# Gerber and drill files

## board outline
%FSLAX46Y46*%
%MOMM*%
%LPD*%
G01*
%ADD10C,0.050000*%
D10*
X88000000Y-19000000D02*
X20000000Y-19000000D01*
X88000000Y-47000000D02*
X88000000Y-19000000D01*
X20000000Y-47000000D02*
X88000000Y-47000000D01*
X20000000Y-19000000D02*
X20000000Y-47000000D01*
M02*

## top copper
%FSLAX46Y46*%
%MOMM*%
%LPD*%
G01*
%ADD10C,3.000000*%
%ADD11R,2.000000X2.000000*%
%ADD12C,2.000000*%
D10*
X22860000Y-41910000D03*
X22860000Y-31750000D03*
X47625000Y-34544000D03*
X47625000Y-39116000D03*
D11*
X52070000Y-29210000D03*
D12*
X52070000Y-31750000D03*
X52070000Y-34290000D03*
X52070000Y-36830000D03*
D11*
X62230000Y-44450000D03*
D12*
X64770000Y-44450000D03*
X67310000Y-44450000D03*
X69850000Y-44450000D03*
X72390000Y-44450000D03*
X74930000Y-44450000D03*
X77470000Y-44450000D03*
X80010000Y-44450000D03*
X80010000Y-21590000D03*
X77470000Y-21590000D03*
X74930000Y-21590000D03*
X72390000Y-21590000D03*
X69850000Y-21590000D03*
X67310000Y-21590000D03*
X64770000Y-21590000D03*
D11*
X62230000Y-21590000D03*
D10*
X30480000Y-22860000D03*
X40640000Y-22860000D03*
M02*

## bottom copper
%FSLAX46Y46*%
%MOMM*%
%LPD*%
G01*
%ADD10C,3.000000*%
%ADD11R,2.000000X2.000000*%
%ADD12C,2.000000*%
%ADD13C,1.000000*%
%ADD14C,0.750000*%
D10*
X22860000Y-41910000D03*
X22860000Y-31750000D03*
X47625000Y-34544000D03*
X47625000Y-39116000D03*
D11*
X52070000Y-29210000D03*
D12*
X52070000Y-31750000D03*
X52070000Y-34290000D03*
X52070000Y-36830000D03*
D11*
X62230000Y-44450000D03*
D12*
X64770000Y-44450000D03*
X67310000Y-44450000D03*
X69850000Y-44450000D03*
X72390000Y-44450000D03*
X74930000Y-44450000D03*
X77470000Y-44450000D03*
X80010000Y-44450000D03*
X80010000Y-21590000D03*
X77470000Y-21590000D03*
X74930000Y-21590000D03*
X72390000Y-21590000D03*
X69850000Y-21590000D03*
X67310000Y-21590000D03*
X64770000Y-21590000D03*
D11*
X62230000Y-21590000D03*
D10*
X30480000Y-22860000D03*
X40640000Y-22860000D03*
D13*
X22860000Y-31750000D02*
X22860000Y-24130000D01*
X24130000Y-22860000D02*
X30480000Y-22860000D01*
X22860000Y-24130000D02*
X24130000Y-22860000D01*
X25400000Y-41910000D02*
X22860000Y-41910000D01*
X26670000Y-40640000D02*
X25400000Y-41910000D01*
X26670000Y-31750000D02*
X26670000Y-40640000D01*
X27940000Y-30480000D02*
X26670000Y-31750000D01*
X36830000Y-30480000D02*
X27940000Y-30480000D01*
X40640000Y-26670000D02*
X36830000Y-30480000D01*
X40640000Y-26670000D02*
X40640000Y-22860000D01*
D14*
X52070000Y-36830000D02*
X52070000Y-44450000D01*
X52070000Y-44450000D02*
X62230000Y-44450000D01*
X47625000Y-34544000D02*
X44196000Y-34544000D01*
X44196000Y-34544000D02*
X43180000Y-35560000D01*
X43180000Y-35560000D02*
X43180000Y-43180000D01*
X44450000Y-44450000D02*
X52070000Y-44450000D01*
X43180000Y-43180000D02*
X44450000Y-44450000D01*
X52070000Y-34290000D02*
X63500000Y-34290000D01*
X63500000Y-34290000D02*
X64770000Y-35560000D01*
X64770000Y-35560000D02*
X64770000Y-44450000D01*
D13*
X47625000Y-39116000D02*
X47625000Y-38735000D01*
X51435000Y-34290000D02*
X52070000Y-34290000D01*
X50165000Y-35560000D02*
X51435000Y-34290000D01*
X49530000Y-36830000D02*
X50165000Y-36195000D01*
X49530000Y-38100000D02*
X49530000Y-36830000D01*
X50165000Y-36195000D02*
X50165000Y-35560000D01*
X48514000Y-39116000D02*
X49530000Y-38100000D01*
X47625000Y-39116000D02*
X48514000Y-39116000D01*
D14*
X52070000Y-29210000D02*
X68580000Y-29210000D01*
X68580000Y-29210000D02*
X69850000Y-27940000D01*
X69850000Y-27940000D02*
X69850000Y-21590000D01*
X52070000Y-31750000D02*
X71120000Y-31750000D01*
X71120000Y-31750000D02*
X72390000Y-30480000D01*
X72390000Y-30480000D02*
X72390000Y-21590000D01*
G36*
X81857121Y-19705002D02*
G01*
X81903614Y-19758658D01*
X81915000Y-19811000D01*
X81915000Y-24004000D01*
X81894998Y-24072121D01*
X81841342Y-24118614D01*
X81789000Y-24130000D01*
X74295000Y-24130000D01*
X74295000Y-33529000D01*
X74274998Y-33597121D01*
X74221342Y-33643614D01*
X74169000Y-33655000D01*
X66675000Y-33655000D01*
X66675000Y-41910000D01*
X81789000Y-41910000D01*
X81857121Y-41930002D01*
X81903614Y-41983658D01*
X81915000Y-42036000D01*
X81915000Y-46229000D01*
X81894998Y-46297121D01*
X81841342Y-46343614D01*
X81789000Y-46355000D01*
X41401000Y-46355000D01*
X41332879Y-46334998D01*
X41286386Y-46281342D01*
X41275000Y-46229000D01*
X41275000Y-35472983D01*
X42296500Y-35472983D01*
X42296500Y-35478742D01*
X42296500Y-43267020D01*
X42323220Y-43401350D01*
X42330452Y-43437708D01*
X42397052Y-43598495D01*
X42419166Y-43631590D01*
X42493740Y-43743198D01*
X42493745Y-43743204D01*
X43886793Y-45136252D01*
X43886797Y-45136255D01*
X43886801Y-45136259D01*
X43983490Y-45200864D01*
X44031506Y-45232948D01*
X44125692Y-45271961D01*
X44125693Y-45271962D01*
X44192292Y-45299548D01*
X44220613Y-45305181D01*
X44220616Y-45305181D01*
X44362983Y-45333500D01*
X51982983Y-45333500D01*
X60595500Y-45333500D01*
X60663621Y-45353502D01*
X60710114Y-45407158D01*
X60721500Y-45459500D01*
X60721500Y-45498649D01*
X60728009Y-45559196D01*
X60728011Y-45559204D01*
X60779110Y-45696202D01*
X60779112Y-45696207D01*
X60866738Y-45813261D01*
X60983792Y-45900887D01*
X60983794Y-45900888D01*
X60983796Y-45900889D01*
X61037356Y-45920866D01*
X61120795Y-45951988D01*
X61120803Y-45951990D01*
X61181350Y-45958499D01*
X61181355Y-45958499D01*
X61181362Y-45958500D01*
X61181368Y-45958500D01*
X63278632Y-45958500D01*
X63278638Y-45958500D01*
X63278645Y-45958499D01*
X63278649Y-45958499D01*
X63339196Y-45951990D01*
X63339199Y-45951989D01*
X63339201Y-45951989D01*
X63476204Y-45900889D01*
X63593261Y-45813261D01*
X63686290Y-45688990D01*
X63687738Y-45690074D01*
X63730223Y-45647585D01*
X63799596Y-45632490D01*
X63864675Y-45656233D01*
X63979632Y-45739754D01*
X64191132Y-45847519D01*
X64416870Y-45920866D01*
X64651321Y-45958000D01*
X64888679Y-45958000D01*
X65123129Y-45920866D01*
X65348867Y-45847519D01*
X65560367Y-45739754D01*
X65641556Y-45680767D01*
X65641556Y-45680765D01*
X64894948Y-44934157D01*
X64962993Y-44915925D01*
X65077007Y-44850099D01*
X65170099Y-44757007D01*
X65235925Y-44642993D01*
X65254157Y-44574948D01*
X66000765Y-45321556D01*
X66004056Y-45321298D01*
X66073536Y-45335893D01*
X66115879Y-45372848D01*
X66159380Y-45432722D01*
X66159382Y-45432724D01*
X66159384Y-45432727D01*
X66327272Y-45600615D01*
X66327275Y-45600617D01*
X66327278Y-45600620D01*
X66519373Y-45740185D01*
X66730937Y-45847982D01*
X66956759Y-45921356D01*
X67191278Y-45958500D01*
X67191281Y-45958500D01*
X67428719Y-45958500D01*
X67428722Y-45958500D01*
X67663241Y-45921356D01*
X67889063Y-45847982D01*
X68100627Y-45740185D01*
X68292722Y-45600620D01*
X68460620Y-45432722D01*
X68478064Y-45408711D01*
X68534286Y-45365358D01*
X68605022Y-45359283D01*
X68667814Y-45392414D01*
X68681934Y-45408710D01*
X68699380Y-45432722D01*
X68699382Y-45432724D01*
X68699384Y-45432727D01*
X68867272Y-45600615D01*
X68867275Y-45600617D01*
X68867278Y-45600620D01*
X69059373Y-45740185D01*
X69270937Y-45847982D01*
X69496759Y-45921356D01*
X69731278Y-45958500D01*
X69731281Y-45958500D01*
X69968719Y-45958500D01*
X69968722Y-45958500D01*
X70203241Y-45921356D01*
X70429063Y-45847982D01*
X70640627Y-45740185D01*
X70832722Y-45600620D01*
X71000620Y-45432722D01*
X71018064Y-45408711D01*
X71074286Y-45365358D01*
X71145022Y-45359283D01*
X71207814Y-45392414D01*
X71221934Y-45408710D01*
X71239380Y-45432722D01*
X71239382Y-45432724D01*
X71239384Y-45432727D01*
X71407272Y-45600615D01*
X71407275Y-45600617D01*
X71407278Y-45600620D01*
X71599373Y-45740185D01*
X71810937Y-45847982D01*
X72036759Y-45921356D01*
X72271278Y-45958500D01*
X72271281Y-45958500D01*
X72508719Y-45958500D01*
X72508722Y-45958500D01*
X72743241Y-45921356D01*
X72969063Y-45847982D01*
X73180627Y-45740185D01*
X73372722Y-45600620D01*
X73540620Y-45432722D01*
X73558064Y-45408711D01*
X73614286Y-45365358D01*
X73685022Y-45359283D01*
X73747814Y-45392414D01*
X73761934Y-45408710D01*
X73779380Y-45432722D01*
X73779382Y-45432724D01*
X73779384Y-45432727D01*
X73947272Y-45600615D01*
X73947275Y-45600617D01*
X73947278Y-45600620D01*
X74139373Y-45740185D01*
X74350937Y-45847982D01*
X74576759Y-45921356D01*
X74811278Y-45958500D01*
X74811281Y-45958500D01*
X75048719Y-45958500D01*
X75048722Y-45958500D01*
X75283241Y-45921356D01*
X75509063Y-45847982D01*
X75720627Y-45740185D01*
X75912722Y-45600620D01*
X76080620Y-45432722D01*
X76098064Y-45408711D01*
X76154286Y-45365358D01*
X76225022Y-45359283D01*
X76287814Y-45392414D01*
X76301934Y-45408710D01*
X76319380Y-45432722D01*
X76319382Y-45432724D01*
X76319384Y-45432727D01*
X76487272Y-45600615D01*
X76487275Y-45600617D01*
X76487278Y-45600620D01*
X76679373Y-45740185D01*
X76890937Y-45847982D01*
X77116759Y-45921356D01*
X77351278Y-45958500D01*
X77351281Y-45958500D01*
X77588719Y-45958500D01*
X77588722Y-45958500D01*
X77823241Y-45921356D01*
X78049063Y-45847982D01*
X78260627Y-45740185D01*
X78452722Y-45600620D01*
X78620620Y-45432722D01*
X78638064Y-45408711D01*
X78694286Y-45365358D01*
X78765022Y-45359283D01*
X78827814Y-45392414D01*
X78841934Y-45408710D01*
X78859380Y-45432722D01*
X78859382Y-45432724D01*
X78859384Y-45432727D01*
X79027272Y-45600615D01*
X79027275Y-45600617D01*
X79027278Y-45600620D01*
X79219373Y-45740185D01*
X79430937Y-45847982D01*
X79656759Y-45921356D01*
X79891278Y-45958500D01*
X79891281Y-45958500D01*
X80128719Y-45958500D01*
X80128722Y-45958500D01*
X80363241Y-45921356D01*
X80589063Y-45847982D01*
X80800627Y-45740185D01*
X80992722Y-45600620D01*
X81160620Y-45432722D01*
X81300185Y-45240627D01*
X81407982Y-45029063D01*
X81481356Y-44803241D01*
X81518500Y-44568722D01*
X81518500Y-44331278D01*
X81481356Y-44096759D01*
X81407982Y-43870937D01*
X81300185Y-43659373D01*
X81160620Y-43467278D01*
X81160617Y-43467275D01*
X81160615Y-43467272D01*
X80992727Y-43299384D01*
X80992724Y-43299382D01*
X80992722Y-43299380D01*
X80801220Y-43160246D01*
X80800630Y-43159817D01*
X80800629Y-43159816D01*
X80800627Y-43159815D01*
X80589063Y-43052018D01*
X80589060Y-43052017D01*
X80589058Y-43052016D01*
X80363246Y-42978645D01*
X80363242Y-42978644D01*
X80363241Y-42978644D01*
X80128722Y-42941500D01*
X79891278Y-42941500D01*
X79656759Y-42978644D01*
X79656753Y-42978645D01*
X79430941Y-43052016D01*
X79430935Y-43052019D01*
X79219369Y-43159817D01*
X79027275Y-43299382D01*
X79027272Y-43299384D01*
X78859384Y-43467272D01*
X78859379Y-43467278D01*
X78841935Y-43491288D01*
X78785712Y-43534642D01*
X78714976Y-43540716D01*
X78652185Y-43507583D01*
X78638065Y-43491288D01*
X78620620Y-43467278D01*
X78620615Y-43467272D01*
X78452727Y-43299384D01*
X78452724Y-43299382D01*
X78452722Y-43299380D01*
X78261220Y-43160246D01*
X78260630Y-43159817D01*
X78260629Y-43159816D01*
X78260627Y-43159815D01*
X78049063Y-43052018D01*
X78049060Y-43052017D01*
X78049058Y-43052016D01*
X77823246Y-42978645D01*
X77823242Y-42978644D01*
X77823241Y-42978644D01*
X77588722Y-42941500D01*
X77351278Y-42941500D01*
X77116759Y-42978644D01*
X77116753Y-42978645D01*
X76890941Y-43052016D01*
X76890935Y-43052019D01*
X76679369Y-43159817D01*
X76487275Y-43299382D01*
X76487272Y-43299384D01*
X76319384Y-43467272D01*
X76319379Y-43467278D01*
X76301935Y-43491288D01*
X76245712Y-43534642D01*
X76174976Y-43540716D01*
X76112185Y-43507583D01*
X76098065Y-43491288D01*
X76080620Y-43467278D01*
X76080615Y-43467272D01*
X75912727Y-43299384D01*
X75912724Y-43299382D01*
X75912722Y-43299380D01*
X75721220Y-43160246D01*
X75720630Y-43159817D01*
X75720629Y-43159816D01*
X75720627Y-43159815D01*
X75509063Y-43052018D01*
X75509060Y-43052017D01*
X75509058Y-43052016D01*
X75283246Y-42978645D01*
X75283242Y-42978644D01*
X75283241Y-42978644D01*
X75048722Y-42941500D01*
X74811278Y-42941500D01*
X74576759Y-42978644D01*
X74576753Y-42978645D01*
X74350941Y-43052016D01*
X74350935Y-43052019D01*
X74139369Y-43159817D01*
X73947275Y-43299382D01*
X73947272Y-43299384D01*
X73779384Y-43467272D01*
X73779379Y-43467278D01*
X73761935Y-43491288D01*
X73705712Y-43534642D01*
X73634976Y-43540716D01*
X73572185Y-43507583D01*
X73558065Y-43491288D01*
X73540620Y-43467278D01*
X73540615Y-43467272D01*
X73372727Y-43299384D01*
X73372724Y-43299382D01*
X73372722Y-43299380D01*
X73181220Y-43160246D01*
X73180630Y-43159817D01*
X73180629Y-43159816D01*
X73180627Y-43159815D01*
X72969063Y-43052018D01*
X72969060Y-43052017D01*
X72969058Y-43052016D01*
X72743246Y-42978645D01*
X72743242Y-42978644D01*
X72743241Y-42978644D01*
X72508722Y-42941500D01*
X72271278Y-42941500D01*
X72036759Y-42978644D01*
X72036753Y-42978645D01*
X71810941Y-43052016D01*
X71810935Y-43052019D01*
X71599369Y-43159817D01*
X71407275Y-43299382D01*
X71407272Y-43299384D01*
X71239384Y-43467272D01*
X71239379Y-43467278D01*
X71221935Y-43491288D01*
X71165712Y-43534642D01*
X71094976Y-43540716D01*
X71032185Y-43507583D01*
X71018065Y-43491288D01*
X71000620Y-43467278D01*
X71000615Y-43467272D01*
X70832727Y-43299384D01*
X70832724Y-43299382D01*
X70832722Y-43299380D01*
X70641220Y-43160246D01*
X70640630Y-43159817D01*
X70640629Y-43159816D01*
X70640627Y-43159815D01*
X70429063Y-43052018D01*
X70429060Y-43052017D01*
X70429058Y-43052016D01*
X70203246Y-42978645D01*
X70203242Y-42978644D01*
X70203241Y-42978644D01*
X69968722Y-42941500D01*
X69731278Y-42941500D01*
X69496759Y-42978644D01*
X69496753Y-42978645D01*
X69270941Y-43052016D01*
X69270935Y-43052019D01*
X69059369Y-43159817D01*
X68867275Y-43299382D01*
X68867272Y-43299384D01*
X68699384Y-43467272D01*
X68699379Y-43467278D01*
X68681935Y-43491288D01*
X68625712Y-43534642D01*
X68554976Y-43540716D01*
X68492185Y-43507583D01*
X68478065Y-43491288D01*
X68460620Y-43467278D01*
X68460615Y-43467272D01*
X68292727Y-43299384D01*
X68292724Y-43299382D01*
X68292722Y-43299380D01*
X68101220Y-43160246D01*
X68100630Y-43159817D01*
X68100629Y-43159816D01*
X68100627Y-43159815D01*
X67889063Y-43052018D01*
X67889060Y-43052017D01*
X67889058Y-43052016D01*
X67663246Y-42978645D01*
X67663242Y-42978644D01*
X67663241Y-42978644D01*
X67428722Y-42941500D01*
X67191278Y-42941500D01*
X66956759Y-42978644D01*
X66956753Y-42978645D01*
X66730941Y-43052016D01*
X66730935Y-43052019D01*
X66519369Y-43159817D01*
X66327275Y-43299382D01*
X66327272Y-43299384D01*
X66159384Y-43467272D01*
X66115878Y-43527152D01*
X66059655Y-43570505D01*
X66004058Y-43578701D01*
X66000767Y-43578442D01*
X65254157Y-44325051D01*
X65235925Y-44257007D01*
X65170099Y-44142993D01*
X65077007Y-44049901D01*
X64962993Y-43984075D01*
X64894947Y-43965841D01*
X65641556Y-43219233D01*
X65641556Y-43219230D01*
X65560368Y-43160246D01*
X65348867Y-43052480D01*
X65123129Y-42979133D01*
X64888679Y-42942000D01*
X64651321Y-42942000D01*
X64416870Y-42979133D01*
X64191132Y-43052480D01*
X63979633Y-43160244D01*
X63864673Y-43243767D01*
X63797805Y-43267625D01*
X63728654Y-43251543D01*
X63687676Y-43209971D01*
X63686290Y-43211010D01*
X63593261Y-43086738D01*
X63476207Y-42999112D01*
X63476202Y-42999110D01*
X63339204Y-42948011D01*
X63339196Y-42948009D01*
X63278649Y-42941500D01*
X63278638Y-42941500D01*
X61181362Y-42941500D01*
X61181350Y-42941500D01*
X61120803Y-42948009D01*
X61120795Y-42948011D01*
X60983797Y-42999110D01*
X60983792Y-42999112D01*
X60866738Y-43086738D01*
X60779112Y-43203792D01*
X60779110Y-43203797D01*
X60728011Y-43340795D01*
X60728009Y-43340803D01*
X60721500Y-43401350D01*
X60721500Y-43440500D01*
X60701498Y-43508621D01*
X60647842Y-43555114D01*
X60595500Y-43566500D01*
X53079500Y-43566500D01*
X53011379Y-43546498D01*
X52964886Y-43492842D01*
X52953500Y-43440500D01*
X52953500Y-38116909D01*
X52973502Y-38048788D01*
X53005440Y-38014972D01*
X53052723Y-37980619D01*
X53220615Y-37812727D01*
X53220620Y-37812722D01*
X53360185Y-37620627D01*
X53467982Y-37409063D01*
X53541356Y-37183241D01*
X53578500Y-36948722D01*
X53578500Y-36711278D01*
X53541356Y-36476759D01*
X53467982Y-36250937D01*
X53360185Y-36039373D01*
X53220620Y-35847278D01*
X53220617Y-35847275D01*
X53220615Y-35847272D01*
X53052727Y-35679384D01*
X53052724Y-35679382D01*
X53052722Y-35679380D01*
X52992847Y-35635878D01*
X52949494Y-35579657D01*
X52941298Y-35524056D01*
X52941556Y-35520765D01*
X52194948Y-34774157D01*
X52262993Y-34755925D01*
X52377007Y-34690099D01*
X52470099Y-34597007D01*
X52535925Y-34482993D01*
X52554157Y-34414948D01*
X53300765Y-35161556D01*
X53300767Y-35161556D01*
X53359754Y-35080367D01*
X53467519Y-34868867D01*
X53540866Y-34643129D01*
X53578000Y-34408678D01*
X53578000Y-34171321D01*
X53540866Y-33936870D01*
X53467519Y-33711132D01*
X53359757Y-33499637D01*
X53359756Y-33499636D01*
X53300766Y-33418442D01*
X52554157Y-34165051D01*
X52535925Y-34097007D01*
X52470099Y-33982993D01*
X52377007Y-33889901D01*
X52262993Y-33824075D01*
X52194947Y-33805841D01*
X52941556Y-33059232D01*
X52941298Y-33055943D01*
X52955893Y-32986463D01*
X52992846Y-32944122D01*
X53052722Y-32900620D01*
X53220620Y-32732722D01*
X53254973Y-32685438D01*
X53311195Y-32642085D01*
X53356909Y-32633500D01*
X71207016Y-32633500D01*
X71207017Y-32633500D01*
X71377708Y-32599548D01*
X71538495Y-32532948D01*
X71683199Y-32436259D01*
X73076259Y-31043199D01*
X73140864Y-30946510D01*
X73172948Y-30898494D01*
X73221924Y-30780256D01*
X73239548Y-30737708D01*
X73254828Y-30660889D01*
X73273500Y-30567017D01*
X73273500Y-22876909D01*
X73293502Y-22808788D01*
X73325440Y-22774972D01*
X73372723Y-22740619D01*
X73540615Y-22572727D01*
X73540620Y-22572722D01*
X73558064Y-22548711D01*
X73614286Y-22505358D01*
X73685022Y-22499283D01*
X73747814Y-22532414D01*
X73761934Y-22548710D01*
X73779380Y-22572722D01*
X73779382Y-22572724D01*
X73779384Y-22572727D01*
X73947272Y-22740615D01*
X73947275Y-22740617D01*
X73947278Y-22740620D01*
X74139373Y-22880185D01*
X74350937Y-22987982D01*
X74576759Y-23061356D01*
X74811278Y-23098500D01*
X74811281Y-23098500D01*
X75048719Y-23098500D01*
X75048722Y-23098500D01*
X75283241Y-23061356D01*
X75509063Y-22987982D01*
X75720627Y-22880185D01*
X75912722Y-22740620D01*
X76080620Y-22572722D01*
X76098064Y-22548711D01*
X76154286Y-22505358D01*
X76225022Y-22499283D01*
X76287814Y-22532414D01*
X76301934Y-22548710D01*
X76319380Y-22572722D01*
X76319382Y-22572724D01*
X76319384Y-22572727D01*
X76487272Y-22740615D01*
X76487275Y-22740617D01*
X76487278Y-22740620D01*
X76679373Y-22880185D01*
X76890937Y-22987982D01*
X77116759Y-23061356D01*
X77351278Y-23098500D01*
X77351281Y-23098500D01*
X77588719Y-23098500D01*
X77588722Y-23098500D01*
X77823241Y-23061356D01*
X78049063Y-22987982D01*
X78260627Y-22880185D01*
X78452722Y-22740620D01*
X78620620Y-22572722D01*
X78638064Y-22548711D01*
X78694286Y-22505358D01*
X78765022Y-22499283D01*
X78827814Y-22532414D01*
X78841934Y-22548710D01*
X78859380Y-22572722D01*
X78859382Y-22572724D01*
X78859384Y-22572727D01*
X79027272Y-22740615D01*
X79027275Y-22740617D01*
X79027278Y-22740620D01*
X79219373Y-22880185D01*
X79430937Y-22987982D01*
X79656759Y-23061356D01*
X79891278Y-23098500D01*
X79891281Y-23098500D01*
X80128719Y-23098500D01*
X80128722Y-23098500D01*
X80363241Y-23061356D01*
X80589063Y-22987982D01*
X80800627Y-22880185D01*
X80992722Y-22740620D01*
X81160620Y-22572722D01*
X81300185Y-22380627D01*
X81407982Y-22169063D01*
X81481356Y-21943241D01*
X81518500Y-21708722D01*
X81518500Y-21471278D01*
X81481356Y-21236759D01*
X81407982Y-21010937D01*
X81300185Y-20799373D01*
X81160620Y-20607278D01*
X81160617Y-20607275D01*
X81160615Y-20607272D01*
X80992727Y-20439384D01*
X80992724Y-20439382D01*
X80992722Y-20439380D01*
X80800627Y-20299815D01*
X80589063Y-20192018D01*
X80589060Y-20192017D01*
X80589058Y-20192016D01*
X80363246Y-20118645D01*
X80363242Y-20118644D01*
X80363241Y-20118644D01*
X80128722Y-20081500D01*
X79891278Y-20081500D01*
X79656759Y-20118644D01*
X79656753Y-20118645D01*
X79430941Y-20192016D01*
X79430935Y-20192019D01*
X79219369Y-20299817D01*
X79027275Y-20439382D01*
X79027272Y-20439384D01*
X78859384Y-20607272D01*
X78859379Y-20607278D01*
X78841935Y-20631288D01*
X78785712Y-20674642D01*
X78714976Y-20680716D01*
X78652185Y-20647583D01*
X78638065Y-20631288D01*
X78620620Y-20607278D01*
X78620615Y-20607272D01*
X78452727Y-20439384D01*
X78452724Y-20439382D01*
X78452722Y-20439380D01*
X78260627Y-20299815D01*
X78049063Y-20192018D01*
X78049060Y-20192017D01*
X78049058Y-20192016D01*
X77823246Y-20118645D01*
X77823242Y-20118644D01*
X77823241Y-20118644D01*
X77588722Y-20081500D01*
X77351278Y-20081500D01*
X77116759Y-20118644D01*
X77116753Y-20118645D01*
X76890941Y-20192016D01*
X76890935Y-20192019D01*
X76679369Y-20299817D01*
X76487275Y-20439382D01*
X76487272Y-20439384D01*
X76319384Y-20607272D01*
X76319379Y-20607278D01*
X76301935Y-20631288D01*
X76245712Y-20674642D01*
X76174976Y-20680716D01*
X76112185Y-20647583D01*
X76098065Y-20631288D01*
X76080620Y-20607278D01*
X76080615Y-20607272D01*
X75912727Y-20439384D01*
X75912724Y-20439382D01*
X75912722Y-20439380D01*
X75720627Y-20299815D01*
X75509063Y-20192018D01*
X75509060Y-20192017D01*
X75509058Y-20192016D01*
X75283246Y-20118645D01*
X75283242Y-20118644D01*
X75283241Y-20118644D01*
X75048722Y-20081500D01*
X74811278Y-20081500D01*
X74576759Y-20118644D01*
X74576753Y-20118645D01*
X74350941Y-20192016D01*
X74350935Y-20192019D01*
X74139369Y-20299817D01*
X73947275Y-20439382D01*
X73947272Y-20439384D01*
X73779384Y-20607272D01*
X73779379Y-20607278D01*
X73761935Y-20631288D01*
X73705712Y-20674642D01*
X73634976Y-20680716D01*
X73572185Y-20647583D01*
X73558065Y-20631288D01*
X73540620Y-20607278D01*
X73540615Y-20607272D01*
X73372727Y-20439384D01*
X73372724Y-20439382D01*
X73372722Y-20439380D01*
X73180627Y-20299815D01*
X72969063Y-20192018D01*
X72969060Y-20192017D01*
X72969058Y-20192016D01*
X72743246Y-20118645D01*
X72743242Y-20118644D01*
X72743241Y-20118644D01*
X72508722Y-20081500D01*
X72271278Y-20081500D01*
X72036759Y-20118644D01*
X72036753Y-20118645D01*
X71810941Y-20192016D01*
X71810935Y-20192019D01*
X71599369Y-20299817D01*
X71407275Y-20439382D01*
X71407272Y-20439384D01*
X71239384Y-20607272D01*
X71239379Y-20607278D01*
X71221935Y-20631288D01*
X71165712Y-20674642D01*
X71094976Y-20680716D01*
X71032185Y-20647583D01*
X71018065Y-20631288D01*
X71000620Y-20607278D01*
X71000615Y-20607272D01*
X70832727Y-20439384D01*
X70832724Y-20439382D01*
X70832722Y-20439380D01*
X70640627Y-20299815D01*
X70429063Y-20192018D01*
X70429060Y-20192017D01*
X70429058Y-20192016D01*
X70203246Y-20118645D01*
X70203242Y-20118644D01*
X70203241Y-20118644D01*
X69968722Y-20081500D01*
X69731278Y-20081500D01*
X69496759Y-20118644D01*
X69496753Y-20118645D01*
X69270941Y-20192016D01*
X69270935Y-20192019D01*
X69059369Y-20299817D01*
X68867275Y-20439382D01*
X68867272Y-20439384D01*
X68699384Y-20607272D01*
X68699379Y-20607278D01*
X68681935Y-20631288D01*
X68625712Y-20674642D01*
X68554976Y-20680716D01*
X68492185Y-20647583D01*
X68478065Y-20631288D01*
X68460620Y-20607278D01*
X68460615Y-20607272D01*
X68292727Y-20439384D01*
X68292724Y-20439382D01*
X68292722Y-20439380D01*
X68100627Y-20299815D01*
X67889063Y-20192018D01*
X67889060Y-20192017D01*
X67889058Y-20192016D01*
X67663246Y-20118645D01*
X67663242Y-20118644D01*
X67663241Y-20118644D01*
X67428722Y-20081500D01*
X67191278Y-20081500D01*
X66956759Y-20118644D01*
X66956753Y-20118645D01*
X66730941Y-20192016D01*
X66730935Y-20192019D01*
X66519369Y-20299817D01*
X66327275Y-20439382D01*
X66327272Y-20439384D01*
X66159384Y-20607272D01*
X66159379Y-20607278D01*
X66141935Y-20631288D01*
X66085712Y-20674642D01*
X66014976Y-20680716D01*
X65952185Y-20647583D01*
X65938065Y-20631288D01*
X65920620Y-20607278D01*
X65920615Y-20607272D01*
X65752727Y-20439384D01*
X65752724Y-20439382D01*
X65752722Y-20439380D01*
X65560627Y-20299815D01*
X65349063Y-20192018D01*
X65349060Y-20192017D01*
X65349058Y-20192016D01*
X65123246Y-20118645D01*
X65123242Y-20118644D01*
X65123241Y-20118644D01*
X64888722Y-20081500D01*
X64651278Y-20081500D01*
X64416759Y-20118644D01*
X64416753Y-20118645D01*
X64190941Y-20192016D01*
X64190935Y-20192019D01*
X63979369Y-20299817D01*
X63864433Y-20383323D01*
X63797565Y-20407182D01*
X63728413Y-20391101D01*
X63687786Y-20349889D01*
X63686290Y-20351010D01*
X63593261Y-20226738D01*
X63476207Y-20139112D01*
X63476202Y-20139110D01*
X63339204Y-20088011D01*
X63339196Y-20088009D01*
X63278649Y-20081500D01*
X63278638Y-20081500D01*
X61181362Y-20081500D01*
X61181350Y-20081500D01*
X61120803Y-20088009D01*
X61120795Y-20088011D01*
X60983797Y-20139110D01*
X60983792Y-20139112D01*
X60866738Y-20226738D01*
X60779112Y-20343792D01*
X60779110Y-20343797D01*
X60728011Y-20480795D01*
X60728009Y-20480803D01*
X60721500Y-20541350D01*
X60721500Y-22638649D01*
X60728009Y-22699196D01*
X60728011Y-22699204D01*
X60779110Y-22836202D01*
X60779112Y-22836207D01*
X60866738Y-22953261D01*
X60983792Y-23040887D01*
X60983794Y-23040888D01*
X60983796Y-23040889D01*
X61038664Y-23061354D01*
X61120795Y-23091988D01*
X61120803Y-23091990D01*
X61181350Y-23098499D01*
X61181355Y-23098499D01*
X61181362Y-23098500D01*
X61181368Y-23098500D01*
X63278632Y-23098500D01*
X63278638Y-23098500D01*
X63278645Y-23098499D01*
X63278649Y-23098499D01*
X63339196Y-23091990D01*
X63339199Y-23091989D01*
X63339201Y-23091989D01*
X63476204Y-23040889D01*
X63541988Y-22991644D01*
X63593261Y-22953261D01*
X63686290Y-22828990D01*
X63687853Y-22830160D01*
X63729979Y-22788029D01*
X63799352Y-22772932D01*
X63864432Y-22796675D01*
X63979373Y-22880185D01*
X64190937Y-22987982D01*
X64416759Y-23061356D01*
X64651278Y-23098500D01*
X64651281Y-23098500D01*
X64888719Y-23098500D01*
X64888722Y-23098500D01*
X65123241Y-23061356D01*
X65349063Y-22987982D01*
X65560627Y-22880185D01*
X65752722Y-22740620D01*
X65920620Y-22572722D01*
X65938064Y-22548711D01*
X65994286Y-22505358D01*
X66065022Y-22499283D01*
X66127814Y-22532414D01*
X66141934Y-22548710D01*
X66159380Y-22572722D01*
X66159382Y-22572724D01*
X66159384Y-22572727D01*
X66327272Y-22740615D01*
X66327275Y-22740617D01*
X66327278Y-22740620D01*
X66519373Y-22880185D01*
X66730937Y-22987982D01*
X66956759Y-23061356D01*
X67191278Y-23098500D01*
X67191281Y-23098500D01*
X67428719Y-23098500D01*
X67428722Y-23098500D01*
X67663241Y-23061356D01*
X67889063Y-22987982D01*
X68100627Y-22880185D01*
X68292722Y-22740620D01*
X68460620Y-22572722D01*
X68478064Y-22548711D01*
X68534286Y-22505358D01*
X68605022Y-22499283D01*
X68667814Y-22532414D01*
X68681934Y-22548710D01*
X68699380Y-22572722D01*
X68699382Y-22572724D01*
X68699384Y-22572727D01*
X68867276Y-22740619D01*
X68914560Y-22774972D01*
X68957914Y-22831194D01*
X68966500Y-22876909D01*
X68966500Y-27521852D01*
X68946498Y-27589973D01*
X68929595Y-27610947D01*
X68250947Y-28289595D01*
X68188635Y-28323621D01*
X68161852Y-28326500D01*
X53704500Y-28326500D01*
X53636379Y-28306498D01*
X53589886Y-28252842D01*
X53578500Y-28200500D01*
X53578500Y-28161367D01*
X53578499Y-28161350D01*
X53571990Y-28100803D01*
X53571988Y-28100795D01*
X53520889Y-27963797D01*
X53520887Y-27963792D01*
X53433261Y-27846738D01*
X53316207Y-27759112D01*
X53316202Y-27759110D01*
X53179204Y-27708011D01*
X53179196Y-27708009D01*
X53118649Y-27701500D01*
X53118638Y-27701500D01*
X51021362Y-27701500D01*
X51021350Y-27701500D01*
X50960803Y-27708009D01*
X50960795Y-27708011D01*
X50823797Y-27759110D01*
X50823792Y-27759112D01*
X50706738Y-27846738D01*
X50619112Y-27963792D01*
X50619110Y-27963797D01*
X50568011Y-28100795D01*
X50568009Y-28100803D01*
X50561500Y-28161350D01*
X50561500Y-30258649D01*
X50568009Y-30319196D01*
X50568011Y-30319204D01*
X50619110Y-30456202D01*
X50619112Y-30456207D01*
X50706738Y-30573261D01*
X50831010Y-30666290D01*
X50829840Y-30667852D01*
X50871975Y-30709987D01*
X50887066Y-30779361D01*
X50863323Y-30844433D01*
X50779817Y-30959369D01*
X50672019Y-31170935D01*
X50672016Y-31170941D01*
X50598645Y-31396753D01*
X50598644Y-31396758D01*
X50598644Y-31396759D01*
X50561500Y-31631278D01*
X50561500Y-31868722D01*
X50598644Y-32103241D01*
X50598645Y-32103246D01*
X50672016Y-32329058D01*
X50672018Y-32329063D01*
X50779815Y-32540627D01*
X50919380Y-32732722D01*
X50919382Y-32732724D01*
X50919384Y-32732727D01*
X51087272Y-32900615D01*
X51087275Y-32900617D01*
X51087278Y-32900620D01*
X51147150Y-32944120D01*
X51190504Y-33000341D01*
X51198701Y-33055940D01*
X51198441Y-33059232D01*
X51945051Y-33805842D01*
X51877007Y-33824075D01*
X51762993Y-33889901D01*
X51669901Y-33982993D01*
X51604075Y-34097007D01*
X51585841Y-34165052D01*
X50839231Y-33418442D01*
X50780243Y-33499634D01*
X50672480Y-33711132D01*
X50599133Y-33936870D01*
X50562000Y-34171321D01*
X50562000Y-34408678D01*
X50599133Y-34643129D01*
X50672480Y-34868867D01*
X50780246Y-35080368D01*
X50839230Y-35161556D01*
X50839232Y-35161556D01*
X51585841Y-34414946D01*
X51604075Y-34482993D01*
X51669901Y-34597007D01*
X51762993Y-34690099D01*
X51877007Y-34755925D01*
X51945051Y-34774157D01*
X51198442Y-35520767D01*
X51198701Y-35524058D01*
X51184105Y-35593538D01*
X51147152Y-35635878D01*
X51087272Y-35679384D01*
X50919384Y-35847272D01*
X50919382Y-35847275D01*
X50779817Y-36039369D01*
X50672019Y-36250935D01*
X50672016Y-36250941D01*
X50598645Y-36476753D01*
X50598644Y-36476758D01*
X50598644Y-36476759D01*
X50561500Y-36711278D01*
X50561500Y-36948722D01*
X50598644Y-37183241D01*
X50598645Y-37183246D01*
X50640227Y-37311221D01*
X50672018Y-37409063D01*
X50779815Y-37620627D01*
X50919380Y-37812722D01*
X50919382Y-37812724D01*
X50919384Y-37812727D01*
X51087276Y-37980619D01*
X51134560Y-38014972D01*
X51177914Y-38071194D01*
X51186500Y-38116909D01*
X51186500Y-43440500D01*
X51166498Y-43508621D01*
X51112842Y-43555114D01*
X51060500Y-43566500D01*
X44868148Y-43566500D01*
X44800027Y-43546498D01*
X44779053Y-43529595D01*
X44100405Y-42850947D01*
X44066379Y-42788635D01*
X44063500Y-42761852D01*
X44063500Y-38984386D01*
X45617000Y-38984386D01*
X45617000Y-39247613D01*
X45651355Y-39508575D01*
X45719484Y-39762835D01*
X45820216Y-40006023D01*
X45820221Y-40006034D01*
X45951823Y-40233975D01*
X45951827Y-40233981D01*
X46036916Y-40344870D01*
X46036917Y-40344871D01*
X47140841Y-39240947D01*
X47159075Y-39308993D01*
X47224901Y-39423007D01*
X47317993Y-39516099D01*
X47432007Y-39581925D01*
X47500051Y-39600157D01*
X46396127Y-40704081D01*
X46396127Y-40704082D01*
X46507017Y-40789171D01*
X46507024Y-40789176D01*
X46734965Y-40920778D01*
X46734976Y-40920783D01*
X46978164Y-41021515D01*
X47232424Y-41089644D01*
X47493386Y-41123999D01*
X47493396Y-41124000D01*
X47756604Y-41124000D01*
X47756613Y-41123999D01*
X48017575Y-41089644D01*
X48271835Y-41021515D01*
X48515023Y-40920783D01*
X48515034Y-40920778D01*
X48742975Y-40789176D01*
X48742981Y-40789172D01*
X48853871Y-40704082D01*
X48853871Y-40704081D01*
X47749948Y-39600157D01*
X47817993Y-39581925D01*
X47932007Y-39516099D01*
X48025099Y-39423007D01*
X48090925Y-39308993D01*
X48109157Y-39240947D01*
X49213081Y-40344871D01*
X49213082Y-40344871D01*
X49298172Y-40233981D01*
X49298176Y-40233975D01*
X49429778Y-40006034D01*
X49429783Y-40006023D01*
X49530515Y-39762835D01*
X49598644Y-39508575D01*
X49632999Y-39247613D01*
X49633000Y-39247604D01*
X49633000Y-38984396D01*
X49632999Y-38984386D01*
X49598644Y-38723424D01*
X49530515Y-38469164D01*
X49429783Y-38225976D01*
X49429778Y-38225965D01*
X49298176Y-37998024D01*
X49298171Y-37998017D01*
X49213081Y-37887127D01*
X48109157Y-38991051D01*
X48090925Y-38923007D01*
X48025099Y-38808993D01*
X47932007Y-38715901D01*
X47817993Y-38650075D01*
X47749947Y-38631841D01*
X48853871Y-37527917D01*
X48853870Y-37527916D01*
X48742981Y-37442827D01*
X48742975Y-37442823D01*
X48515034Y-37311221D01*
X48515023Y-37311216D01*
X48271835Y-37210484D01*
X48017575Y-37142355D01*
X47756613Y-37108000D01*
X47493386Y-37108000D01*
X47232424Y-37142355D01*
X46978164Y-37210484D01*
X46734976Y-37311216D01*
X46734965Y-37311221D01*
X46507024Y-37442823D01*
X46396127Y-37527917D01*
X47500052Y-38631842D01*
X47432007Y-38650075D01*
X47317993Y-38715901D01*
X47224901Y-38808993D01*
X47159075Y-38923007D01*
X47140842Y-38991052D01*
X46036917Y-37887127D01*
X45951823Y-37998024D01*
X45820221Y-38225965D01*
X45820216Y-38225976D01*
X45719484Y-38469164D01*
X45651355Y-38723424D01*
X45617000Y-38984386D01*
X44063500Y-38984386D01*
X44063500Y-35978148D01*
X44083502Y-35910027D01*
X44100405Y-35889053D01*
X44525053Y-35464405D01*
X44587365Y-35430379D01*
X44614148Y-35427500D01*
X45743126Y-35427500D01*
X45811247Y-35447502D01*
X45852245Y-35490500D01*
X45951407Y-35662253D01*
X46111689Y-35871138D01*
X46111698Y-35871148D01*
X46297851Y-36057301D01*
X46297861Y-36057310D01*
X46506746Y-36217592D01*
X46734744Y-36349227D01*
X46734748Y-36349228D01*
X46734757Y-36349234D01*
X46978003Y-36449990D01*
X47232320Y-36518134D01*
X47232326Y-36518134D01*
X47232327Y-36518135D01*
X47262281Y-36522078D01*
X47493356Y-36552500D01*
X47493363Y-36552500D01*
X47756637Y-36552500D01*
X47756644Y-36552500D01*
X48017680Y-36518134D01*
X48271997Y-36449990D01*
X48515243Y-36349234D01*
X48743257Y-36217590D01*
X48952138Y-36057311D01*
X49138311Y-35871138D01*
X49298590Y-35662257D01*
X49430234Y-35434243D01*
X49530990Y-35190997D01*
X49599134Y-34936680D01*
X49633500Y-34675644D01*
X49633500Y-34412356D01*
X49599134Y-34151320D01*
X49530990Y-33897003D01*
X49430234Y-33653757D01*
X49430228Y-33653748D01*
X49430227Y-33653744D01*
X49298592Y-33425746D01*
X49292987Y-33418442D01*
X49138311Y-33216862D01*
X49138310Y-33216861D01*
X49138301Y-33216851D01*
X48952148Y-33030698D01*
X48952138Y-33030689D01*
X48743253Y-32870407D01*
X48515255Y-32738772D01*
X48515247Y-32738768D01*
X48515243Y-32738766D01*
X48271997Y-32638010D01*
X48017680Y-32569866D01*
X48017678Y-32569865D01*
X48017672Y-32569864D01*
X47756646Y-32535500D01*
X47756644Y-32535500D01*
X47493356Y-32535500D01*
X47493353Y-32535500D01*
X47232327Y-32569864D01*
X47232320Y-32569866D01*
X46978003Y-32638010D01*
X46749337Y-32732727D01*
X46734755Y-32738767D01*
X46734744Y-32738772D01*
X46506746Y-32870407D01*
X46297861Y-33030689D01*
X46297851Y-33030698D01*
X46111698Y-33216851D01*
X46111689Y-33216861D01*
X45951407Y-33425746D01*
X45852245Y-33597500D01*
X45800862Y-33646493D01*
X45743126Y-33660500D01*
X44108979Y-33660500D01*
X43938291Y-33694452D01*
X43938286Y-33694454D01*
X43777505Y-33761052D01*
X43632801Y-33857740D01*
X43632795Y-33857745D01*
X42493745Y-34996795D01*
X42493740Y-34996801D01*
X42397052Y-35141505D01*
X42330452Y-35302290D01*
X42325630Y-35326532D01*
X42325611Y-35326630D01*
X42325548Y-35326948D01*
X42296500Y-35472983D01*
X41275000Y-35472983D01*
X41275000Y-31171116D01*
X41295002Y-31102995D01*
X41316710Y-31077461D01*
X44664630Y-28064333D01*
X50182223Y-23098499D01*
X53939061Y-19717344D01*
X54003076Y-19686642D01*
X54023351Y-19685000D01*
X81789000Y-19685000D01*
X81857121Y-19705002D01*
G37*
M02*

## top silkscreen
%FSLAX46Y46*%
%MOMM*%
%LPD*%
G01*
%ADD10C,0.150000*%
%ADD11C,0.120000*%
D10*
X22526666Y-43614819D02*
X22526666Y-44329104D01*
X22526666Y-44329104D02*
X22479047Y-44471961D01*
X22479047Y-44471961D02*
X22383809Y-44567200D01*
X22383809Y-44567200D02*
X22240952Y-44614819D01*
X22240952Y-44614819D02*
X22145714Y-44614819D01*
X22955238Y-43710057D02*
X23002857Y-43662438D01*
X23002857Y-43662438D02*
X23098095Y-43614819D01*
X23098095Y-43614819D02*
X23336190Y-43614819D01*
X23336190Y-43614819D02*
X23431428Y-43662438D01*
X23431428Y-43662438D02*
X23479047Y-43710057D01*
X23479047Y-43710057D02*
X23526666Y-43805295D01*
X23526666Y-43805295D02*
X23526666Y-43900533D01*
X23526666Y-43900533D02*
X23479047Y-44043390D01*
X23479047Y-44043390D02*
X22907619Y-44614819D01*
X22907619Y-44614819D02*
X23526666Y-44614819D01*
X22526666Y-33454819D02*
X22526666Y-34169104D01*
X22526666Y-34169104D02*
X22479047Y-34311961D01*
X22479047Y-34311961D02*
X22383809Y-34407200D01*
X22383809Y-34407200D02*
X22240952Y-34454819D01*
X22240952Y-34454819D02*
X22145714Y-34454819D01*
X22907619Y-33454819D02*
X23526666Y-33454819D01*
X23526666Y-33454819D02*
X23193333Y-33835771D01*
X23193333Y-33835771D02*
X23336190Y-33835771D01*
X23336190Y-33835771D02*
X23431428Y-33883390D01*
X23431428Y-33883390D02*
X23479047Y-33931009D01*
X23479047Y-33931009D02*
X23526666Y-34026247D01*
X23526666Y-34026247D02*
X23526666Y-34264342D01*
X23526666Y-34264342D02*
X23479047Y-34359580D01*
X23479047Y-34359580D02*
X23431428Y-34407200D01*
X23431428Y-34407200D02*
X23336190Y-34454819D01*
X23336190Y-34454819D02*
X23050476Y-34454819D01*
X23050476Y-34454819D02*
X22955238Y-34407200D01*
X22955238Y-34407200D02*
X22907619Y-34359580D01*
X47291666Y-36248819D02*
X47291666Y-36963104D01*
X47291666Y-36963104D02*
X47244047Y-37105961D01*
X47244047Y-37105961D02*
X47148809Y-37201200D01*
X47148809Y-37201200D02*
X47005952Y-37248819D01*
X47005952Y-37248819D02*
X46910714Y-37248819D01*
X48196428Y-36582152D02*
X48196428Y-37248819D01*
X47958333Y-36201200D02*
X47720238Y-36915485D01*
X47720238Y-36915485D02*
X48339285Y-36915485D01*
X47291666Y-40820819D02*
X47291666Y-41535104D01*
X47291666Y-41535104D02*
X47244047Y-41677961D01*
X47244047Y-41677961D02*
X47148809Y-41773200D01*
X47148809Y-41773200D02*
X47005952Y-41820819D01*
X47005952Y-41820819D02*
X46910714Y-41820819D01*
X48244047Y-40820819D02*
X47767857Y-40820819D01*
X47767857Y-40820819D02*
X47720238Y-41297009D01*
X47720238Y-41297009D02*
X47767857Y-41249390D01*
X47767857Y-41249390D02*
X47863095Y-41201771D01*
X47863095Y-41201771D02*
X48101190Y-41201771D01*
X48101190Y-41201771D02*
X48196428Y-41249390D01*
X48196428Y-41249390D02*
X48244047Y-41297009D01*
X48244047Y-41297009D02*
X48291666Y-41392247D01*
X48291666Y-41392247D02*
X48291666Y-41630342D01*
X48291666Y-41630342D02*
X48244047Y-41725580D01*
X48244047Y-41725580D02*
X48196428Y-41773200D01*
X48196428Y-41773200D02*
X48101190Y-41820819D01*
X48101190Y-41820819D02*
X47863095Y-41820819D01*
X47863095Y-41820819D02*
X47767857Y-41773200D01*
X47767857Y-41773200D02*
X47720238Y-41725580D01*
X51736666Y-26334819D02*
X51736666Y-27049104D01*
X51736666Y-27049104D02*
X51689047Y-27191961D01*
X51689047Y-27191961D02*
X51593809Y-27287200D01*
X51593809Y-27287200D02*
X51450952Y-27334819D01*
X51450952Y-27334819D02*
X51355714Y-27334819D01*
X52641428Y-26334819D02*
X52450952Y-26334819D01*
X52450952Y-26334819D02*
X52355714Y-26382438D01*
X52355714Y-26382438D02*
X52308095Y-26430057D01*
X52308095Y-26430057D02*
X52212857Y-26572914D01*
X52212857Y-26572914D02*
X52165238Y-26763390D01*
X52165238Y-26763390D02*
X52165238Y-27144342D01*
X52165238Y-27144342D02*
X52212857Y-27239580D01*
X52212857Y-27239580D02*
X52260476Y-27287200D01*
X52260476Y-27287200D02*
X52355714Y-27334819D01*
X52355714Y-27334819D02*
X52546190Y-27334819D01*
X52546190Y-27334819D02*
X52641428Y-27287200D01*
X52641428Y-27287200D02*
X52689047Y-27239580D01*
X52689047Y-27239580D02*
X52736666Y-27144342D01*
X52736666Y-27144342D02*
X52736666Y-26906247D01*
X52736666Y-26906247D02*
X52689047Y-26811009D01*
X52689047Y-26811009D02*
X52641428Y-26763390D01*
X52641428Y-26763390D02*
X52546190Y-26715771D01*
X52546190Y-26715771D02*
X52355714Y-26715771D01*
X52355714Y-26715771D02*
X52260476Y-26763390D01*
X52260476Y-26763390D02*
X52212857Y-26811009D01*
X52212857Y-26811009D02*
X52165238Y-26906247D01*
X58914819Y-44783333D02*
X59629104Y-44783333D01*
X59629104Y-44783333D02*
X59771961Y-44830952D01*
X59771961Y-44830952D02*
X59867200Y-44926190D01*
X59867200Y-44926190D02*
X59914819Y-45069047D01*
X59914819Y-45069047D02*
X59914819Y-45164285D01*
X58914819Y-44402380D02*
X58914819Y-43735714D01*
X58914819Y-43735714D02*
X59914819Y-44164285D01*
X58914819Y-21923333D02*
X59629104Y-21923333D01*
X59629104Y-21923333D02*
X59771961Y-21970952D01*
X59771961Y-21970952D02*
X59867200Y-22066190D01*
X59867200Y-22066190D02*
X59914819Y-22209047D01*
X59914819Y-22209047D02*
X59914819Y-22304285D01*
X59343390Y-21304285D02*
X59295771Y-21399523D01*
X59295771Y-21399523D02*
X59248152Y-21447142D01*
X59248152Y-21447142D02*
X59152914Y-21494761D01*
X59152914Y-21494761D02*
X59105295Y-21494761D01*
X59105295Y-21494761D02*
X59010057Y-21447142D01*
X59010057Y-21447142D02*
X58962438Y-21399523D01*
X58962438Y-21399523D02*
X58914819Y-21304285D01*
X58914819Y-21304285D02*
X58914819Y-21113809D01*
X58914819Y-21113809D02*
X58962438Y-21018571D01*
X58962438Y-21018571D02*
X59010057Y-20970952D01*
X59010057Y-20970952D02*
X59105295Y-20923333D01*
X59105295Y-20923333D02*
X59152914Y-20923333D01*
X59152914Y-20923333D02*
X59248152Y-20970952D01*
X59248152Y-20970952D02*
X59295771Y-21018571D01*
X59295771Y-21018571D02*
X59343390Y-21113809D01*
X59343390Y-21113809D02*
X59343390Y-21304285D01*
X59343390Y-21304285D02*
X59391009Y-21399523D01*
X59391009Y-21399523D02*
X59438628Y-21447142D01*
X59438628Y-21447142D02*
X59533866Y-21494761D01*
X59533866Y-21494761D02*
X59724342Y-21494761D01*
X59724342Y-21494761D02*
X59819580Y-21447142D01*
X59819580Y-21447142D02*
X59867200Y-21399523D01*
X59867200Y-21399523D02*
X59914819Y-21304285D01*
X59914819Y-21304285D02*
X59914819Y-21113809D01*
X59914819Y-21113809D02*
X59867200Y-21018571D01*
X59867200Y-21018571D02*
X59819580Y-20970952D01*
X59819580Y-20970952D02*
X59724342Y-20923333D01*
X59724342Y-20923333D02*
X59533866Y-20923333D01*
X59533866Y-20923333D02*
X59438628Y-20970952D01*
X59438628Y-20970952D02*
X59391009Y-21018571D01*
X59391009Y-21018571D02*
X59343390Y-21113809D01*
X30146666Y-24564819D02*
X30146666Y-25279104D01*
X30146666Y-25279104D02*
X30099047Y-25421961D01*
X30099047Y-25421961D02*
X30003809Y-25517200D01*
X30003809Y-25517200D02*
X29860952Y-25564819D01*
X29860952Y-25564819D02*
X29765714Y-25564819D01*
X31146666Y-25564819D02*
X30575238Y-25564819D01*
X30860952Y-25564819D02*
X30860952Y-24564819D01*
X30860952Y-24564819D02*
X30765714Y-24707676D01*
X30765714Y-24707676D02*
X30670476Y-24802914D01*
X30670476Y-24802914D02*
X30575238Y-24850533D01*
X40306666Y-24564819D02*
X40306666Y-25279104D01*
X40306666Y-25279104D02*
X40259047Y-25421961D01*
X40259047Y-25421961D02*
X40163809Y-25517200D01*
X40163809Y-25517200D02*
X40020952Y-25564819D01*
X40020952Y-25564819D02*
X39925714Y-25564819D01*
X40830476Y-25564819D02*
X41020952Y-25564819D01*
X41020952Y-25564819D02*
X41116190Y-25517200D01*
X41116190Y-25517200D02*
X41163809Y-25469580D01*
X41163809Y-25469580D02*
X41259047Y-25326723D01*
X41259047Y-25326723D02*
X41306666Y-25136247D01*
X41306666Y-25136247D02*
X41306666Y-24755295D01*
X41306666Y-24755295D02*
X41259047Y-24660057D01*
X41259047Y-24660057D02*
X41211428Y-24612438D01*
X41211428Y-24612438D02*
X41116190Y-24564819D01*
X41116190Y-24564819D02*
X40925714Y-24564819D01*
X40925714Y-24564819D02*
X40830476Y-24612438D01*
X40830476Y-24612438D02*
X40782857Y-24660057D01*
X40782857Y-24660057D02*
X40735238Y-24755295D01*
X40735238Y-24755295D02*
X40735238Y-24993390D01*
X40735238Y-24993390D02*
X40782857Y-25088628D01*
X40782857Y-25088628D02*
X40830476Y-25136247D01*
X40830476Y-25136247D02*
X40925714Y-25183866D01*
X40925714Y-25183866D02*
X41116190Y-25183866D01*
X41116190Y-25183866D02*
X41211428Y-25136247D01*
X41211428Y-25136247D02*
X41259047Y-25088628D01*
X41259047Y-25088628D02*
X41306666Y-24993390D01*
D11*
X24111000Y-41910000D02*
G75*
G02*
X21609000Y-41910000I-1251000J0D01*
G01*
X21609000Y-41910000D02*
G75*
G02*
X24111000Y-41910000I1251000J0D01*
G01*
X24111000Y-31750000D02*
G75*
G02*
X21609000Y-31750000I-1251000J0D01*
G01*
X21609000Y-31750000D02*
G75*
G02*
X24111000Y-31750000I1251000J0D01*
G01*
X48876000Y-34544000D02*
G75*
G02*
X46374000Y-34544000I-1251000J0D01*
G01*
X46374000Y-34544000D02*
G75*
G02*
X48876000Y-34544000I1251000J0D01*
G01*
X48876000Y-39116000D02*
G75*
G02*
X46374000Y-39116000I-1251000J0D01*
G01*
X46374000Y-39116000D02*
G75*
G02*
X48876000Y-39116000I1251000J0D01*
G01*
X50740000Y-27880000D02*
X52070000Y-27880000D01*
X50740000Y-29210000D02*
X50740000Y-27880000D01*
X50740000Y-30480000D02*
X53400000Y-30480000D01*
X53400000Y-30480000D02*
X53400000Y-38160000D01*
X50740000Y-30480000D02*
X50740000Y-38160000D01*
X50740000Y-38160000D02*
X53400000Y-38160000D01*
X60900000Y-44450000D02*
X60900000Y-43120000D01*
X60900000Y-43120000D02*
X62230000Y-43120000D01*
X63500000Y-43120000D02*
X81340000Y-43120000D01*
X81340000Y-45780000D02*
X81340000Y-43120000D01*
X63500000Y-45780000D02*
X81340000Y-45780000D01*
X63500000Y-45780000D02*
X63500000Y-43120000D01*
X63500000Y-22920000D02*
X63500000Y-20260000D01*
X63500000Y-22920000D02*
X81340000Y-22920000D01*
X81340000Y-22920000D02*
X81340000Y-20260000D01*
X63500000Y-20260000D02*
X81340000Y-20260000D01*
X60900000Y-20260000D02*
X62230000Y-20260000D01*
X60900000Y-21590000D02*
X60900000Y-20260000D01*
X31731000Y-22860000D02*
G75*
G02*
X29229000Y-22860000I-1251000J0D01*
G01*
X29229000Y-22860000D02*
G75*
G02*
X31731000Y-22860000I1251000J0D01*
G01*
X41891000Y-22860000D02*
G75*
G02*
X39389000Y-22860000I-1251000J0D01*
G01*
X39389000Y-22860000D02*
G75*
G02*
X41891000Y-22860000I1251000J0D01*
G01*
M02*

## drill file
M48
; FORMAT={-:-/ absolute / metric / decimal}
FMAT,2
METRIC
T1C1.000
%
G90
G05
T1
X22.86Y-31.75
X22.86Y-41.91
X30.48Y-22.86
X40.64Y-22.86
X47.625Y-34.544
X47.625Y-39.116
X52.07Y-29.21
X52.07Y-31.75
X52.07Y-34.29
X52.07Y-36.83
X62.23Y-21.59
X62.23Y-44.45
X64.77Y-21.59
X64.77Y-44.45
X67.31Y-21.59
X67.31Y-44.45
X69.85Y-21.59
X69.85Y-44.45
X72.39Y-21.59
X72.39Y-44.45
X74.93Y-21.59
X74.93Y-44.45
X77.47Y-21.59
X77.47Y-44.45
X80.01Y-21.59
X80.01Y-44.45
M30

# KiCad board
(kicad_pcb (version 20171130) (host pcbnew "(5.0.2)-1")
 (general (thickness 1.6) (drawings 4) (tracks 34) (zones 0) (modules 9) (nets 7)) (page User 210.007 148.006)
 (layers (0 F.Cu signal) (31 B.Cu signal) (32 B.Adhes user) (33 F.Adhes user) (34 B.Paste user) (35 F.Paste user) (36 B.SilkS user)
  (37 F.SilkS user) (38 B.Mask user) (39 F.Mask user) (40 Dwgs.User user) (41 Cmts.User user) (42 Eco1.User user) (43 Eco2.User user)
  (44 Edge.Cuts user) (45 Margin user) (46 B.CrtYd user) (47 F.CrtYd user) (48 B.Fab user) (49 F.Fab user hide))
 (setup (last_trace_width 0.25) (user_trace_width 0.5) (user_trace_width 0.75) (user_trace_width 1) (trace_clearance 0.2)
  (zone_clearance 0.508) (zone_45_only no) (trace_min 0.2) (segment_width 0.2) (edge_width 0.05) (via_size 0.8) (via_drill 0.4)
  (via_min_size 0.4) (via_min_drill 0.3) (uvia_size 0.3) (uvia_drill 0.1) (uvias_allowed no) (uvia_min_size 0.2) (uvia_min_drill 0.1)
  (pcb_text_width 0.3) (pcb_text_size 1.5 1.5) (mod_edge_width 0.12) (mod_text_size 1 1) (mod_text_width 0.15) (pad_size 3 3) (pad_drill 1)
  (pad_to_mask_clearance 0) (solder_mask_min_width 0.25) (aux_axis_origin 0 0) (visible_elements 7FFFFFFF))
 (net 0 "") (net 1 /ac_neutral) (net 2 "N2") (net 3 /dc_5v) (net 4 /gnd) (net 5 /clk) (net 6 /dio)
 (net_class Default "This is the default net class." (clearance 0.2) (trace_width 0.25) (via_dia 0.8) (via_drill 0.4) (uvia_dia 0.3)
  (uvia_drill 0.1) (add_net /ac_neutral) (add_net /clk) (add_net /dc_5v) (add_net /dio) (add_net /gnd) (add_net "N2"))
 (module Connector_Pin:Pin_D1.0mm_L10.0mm (layer F.Cu) (at 22.86 41.91)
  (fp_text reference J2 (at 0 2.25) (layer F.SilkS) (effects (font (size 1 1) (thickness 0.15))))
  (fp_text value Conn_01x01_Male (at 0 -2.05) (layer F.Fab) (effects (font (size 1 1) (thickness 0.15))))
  (fp_circle (center 0 0) (end 1.25 0.05) (layer F.SilkS) (width 0.12))
  (pad 1 thru_hole circle (at 0 0) (size 3 3) (drill 1) (layers *.Cu *.Mask) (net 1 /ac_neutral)))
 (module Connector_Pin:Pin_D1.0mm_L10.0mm (layer F.Cu) (at 22.86 31.75)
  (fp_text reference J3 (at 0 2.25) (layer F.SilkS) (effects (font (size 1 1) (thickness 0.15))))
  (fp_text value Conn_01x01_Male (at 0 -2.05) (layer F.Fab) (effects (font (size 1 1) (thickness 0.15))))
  (fp_circle (center 0 0) (end 1.25 0.05) (layer F.SilkS) (width 0.12))
  (pad 1 thru_hole circle (at 0 0) (size 3 3) (drill 1) (layers *.Cu *.Mask) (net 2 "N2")))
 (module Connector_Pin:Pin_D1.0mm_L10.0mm (layer F.Cu) (at 47.625 34.544)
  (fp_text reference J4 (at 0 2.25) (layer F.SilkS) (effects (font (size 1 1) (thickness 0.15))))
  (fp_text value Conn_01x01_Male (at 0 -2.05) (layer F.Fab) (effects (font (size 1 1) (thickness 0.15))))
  (fp_circle (center 0 0) (end 1.25 0.05) (layer F.SilkS) (width 0.12))
  (pad 1 thru_hole circle (at 0 0) (size 3 3) (drill 1) (layers *.Cu *.Mask) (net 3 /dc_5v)))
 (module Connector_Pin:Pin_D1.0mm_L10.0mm (layer F.Cu) (at 47.625 39.116)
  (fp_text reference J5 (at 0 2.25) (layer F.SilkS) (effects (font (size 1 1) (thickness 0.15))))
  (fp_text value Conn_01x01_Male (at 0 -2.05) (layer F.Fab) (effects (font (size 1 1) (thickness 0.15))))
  (fp_circle (center 0 0) (end 1.25 0.05) (layer F.SilkS) (width 0.12))
  (pad 1 thru_hole circle (at 0 0) (size 3 3) (drill 1) (layers *.Cu *.Mask) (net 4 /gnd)))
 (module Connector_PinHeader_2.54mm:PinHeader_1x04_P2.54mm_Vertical (layer F.Cu) (at 52.07 29.21)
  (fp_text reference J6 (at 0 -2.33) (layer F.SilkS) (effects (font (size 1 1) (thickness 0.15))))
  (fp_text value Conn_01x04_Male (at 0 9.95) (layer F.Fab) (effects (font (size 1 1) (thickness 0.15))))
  (fp_line (start -1.33 -1.33) (end 0 -1.33) (layer F.SilkS) (width 0.12))
  (fp_line (start -1.33 0) (end -1.33 -1.33) (layer F.SilkS) (width 0.12))
  (fp_line (start -1.33 1.27) (end 1.33 1.27) (layer F.SilkS) (width 0.12))
  (fp_line (start 1.33 1.27) (end 1.33 8.95) (layer F.SilkS) (width 0.12))
  (fp_line (start -1.33 1.27) (end -1.33 8.95) (layer F.SilkS) (width 0.12))
  (fp_line (start -1.33 8.95) (end 1.33 8.95) (layer F.SilkS) (width 0.12))
  (pad 1 thru_hole rect (at 0 0) (size 2 2) (drill 1) (layers *.Cu *.Mask) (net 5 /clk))
  (pad 2 thru_hole circle (at 0 2.54) (size 2 2) (drill 1) (layers *.Cu *.Mask) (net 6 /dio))
  (pad 3 thru_hole circle (at 0 5.08) (size 2 2) (drill 1) (layers *.Cu *.Mask) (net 4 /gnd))
  (pad 4 thru_hole circle (at 0 7.62) (size 2 2) (drill 1) (layers *.Cu *.Mask) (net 3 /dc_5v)))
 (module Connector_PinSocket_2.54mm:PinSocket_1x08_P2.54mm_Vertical (layer F.Cu) (at 62.23 44.45 90)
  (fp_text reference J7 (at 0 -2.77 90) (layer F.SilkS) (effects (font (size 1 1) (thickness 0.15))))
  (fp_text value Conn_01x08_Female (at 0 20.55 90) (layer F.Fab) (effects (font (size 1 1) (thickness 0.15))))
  (fp_line (start 0 -1.33) (end 1.33 -1.33) (layer F.SilkS) (width 0.12))
  (fp_line (start 1.33 -1.33) (end 1.33 0) (layer F.SilkS) (width 0.12))
  (fp_line (start 1.33 1.27) (end 1.33 19.11) (layer F.SilkS) (width 0.12))
  (fp_line (start -1.33 19.11) (end 1.33 19.11) (layer F.SilkS) (width 0.12))
  (fp_line (start -1.33 1.27) (end -1.33 19.11) (layer F.SilkS) (width 0.12))
  (fp_line (start -1.33 1.27) (end 1.33 1.27) (layer F.SilkS) (width 0.12))
  (pad 1 thru_hole rect (at 0 0 90) (size 2 2) (drill 1) (layers *.Cu *.Mask) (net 3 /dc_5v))
  (pad 2 thru_hole circle (at 0 2.54 90) (size 2 2) (drill 1) (layers *.Cu *.Mask) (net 4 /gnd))
  (pad 3 thru_hole circle (at 0 5.08 90) (size 2 2) (drill 1) (layers *.Cu *.Mask))
  (pad 4 thru_hole circle (at 0 7.62 90) (size 2 2) (drill 1) (layers *.Cu *.Mask))
  (pad 5 thru_hole circle (at 0 10.16 90) (size 2 2) (drill 1) (layers *.Cu *.Mask))
  (pad 6 thru_hole circle (at 0 12.7 90) (size 2 2) (drill 1) (layers *.Cu *.Mask))
  (pad 7 thru_hole circle (at 0 15.24 90) (size 2 2) (drill 1) (layers *.Cu *.Mask))
  (pad 8 thru_hole circle (at 0 17.78 90) (size 2 2) (drill 1) (layers *.Cu *.Mask)))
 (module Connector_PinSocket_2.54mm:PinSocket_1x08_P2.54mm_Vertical (layer F.Cu) (at 62.23 21.59 90)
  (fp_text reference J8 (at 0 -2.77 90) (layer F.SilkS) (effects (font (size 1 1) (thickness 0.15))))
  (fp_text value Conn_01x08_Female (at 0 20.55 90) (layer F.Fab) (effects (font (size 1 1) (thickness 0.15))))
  (fp_line (start -1.33 1.27) (end 1.33 1.27) (layer F.SilkS) (width 0.12))
  (fp_line (start -1.33 1.27) (end -1.33 19.11) (layer F.SilkS) (width 0.12))
  (fp_line (start -1.33 19.11) (end 1.33 19.11) (layer F.SilkS) (width 0.12))
  (fp_line (start 1.33 1.27) (end 1.33 19.11) (layer F.SilkS) (width 0.12))
  (fp_line (start 1.33 -1.33) (end 1.33 0) (layer F.SilkS) (width 0.12))
  (fp_line (start 0 -1.33) (end 1.33 -1.33) (layer F.SilkS) (width 0.12))
  (pad 8 thru_hole circle (at 0 17.78 90) (size 2 2) (drill 1) (layers *.Cu *.Mask))
  (pad 7 thru_hole circle (at 0 15.24 90) (size 2 2) (drill 1) (layers *.Cu *.Mask))
  (pad 6 thru_hole circle (at 0 12.7 90) (size 2 2) (drill 1) (layers *.Cu *.Mask))
  (pad 5 thru_hole circle (at 0 10.16 90) (size 2 2) (drill 1) (layers *.Cu *.Mask) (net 6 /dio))
  (pad 4 thru_hole circle (at 0 7.62 90) (size 2 2) (drill 1) (layers *.Cu *.Mask) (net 5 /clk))
  (pad 3 thru_hole circle (at 0 5.08 90) (size 2 2) (drill 1) (layers *.Cu *.Mask))
  (pad 2 thru_hole circle (at 0 2.54 90) (size 2 2) (drill 1) (layers *.Cu *.Mask))
  (pad 1 thru_hole rect (at 0 0 90) (size 2 2) (drill 1) (layers *.Cu *.Mask)))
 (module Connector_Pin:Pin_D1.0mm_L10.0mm (layer F.Cu) (at 30.48 22.86)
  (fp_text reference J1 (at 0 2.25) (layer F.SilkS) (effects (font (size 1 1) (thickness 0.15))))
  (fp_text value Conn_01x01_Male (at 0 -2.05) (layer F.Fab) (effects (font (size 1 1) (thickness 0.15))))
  (fp_circle (center 0 0) (end 1.25 0.05) (layer F.SilkS) (width 0.12))
  (pad 1 thru_hole circle (at 0 0) (size 3 3) (drill 1) (layers *.Cu *.Mask) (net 2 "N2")))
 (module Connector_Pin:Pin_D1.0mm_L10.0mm (layer F.Cu) (at 40.64 22.86)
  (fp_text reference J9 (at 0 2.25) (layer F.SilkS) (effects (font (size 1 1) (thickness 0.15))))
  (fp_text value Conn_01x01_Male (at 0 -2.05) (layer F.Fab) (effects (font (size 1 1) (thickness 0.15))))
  (fp_circle (center 0 0) (end 1.25 0.05) (layer F.SilkS) (width 0.12))
  (pad 1 thru_hole circle (at 0 0) (size 3 3) (drill 1) (layers *.Cu *.Mask) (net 1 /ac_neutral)))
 (gr_line (start 88 19) (end 20 19) (layer Edge.Cuts) (width 0.05))
 (gr_line (start 88 47) (end 88 19) (layer Edge.Cuts) (width 0.05))
 (gr_line (start 20 47) (end 88 47) (layer Edge.Cuts) (width 0.05))
 (gr_line (start 20 19) (end 20 47) (layer Edge.Cuts) (width 0.05))
 (segment (start 22.86 31.75) (end 22.86 24.13) (width 1) (layer B.Cu) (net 2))
 (segment (start 24.13 22.86) (end 30.48 22.86) (width 1) (layer B.Cu) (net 2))
 (segment (start 22.86 24.13) (end 24.13 22.86) (width 1) (layer B.Cu) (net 2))
 (segment (start 25.4 41.91) (end 22.86 41.91) (width 1) (layer B.Cu) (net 1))
 (segment (start 26.67 40.64) (end 25.4 41.91) (width 1) (layer B.Cu) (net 1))
 (segment (start 26.67 31.75) (end 26.67 40.64) (width 1) (layer B.Cu) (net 1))
 (segment (start 27.94 30.48) (end 26.67 31.75) (width 1) (layer B.Cu) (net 1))
 (segment (start 36.83 30.48) (end 27.94 30.48) (width 1) (layer B.Cu) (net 1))
 (segment (start 40.64 26.67) (end 36.83 30.48) (width 1) (layer B.Cu) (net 1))
 (segment (start 40.64 26.67) (end 40.64 22.86) (width 1) (layer B.Cu) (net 1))
 (segment (start 52.07 36.83) (end 52.07 44.45) (width 0.75) (layer B.Cu) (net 3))
 (segment (start 52.07 44.45) (end 62.23 44.45) (width 0.75) (layer B.Cu) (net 3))
 (segment (start 47.625 34.544) (end 44.196 34.544) (width 0.75) (layer B.Cu) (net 3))
 (segment (start 44.196 34.544) (end 43.18 35.56) (width 0.75) (layer B.Cu) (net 3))
 (segment (start 43.18 35.56) (end 43.18 43.18) (width 0.75) (layer B.Cu) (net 3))
 (segment (start 44.45 44.45) (end 52.07 44.45) (width 0.75) (layer B.Cu) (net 3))
 (segment (start 43.18 43.18) (end 44.45 44.45) (width 0.75) (layer B.Cu) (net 3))
 (segment (start 52.07 34.29) (end 63.5 34.29) (width 0.75) (layer B.Cu) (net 4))
 (segment (start 63.5 34.29) (end 64.77 35.56) (width 0.75) (layer B.Cu) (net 4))
 (segment (start 64.77 35.56) (end 64.77 44.45) (width 0.75) (layer B.Cu) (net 4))
 (segment (start 47.625 39.116) (end 47.625 38.735) (width 1) (layer B.Cu) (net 4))
 (segment (start 51.435 34.29) (end 52.07 34.29) (width 1) (layer B.Cu) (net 4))
 (segment (start 50.165 35.56) (end 51.435 34.29) (width 1) (layer B.Cu) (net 4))
 (segment (start 49.53 36.83) (end 50.165 36.195) (width 1) (layer B.Cu) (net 4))
 (segment (start 49.53 38.1) (end 49.53 36.83) (width 1) (layer B.Cu) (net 4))
 (segment (start 50.165 36.195) (end 50.165 35.56) (width 1) (layer B.Cu) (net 4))
 (segment (start 48.514 39.116) (end 49.53 38.1) (width 1) (layer B.Cu) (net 4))
 (segment (start 47.625 39.116) (end 48.514 39.116) (width 1) (layer B.Cu) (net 4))
 (segment (start 52.07 29.21) (end 68.58 29.21) (width 0.75) (layer B.Cu) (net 5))
 (segment (start 68.58 29.21) (end 69.85 27.94) (width 0.75) (layer B.Cu) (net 5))
 (segment (start 69.85 27.94) (end 69.85 21.59) (width 0.75) (layer B.Cu) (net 5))
 (segment (start 52.07 31.75) (end 71.12 31.75) (width 0.75) (layer B.Cu) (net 6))
 (segment (start 71.12 31.75) (end 72.39 30.48) (width 0.75) (layer B.Cu) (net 6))
 (segment (start 72.39 30.48) (end 72.39 21.59) (width 0.75) (layer B.Cu) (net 6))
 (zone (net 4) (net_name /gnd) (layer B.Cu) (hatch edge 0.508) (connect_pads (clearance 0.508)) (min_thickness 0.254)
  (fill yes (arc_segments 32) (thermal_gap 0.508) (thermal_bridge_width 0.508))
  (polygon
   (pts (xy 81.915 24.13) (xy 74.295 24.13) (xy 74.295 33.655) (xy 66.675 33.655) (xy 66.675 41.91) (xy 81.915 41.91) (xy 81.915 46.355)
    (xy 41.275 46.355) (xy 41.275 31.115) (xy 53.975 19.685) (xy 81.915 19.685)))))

